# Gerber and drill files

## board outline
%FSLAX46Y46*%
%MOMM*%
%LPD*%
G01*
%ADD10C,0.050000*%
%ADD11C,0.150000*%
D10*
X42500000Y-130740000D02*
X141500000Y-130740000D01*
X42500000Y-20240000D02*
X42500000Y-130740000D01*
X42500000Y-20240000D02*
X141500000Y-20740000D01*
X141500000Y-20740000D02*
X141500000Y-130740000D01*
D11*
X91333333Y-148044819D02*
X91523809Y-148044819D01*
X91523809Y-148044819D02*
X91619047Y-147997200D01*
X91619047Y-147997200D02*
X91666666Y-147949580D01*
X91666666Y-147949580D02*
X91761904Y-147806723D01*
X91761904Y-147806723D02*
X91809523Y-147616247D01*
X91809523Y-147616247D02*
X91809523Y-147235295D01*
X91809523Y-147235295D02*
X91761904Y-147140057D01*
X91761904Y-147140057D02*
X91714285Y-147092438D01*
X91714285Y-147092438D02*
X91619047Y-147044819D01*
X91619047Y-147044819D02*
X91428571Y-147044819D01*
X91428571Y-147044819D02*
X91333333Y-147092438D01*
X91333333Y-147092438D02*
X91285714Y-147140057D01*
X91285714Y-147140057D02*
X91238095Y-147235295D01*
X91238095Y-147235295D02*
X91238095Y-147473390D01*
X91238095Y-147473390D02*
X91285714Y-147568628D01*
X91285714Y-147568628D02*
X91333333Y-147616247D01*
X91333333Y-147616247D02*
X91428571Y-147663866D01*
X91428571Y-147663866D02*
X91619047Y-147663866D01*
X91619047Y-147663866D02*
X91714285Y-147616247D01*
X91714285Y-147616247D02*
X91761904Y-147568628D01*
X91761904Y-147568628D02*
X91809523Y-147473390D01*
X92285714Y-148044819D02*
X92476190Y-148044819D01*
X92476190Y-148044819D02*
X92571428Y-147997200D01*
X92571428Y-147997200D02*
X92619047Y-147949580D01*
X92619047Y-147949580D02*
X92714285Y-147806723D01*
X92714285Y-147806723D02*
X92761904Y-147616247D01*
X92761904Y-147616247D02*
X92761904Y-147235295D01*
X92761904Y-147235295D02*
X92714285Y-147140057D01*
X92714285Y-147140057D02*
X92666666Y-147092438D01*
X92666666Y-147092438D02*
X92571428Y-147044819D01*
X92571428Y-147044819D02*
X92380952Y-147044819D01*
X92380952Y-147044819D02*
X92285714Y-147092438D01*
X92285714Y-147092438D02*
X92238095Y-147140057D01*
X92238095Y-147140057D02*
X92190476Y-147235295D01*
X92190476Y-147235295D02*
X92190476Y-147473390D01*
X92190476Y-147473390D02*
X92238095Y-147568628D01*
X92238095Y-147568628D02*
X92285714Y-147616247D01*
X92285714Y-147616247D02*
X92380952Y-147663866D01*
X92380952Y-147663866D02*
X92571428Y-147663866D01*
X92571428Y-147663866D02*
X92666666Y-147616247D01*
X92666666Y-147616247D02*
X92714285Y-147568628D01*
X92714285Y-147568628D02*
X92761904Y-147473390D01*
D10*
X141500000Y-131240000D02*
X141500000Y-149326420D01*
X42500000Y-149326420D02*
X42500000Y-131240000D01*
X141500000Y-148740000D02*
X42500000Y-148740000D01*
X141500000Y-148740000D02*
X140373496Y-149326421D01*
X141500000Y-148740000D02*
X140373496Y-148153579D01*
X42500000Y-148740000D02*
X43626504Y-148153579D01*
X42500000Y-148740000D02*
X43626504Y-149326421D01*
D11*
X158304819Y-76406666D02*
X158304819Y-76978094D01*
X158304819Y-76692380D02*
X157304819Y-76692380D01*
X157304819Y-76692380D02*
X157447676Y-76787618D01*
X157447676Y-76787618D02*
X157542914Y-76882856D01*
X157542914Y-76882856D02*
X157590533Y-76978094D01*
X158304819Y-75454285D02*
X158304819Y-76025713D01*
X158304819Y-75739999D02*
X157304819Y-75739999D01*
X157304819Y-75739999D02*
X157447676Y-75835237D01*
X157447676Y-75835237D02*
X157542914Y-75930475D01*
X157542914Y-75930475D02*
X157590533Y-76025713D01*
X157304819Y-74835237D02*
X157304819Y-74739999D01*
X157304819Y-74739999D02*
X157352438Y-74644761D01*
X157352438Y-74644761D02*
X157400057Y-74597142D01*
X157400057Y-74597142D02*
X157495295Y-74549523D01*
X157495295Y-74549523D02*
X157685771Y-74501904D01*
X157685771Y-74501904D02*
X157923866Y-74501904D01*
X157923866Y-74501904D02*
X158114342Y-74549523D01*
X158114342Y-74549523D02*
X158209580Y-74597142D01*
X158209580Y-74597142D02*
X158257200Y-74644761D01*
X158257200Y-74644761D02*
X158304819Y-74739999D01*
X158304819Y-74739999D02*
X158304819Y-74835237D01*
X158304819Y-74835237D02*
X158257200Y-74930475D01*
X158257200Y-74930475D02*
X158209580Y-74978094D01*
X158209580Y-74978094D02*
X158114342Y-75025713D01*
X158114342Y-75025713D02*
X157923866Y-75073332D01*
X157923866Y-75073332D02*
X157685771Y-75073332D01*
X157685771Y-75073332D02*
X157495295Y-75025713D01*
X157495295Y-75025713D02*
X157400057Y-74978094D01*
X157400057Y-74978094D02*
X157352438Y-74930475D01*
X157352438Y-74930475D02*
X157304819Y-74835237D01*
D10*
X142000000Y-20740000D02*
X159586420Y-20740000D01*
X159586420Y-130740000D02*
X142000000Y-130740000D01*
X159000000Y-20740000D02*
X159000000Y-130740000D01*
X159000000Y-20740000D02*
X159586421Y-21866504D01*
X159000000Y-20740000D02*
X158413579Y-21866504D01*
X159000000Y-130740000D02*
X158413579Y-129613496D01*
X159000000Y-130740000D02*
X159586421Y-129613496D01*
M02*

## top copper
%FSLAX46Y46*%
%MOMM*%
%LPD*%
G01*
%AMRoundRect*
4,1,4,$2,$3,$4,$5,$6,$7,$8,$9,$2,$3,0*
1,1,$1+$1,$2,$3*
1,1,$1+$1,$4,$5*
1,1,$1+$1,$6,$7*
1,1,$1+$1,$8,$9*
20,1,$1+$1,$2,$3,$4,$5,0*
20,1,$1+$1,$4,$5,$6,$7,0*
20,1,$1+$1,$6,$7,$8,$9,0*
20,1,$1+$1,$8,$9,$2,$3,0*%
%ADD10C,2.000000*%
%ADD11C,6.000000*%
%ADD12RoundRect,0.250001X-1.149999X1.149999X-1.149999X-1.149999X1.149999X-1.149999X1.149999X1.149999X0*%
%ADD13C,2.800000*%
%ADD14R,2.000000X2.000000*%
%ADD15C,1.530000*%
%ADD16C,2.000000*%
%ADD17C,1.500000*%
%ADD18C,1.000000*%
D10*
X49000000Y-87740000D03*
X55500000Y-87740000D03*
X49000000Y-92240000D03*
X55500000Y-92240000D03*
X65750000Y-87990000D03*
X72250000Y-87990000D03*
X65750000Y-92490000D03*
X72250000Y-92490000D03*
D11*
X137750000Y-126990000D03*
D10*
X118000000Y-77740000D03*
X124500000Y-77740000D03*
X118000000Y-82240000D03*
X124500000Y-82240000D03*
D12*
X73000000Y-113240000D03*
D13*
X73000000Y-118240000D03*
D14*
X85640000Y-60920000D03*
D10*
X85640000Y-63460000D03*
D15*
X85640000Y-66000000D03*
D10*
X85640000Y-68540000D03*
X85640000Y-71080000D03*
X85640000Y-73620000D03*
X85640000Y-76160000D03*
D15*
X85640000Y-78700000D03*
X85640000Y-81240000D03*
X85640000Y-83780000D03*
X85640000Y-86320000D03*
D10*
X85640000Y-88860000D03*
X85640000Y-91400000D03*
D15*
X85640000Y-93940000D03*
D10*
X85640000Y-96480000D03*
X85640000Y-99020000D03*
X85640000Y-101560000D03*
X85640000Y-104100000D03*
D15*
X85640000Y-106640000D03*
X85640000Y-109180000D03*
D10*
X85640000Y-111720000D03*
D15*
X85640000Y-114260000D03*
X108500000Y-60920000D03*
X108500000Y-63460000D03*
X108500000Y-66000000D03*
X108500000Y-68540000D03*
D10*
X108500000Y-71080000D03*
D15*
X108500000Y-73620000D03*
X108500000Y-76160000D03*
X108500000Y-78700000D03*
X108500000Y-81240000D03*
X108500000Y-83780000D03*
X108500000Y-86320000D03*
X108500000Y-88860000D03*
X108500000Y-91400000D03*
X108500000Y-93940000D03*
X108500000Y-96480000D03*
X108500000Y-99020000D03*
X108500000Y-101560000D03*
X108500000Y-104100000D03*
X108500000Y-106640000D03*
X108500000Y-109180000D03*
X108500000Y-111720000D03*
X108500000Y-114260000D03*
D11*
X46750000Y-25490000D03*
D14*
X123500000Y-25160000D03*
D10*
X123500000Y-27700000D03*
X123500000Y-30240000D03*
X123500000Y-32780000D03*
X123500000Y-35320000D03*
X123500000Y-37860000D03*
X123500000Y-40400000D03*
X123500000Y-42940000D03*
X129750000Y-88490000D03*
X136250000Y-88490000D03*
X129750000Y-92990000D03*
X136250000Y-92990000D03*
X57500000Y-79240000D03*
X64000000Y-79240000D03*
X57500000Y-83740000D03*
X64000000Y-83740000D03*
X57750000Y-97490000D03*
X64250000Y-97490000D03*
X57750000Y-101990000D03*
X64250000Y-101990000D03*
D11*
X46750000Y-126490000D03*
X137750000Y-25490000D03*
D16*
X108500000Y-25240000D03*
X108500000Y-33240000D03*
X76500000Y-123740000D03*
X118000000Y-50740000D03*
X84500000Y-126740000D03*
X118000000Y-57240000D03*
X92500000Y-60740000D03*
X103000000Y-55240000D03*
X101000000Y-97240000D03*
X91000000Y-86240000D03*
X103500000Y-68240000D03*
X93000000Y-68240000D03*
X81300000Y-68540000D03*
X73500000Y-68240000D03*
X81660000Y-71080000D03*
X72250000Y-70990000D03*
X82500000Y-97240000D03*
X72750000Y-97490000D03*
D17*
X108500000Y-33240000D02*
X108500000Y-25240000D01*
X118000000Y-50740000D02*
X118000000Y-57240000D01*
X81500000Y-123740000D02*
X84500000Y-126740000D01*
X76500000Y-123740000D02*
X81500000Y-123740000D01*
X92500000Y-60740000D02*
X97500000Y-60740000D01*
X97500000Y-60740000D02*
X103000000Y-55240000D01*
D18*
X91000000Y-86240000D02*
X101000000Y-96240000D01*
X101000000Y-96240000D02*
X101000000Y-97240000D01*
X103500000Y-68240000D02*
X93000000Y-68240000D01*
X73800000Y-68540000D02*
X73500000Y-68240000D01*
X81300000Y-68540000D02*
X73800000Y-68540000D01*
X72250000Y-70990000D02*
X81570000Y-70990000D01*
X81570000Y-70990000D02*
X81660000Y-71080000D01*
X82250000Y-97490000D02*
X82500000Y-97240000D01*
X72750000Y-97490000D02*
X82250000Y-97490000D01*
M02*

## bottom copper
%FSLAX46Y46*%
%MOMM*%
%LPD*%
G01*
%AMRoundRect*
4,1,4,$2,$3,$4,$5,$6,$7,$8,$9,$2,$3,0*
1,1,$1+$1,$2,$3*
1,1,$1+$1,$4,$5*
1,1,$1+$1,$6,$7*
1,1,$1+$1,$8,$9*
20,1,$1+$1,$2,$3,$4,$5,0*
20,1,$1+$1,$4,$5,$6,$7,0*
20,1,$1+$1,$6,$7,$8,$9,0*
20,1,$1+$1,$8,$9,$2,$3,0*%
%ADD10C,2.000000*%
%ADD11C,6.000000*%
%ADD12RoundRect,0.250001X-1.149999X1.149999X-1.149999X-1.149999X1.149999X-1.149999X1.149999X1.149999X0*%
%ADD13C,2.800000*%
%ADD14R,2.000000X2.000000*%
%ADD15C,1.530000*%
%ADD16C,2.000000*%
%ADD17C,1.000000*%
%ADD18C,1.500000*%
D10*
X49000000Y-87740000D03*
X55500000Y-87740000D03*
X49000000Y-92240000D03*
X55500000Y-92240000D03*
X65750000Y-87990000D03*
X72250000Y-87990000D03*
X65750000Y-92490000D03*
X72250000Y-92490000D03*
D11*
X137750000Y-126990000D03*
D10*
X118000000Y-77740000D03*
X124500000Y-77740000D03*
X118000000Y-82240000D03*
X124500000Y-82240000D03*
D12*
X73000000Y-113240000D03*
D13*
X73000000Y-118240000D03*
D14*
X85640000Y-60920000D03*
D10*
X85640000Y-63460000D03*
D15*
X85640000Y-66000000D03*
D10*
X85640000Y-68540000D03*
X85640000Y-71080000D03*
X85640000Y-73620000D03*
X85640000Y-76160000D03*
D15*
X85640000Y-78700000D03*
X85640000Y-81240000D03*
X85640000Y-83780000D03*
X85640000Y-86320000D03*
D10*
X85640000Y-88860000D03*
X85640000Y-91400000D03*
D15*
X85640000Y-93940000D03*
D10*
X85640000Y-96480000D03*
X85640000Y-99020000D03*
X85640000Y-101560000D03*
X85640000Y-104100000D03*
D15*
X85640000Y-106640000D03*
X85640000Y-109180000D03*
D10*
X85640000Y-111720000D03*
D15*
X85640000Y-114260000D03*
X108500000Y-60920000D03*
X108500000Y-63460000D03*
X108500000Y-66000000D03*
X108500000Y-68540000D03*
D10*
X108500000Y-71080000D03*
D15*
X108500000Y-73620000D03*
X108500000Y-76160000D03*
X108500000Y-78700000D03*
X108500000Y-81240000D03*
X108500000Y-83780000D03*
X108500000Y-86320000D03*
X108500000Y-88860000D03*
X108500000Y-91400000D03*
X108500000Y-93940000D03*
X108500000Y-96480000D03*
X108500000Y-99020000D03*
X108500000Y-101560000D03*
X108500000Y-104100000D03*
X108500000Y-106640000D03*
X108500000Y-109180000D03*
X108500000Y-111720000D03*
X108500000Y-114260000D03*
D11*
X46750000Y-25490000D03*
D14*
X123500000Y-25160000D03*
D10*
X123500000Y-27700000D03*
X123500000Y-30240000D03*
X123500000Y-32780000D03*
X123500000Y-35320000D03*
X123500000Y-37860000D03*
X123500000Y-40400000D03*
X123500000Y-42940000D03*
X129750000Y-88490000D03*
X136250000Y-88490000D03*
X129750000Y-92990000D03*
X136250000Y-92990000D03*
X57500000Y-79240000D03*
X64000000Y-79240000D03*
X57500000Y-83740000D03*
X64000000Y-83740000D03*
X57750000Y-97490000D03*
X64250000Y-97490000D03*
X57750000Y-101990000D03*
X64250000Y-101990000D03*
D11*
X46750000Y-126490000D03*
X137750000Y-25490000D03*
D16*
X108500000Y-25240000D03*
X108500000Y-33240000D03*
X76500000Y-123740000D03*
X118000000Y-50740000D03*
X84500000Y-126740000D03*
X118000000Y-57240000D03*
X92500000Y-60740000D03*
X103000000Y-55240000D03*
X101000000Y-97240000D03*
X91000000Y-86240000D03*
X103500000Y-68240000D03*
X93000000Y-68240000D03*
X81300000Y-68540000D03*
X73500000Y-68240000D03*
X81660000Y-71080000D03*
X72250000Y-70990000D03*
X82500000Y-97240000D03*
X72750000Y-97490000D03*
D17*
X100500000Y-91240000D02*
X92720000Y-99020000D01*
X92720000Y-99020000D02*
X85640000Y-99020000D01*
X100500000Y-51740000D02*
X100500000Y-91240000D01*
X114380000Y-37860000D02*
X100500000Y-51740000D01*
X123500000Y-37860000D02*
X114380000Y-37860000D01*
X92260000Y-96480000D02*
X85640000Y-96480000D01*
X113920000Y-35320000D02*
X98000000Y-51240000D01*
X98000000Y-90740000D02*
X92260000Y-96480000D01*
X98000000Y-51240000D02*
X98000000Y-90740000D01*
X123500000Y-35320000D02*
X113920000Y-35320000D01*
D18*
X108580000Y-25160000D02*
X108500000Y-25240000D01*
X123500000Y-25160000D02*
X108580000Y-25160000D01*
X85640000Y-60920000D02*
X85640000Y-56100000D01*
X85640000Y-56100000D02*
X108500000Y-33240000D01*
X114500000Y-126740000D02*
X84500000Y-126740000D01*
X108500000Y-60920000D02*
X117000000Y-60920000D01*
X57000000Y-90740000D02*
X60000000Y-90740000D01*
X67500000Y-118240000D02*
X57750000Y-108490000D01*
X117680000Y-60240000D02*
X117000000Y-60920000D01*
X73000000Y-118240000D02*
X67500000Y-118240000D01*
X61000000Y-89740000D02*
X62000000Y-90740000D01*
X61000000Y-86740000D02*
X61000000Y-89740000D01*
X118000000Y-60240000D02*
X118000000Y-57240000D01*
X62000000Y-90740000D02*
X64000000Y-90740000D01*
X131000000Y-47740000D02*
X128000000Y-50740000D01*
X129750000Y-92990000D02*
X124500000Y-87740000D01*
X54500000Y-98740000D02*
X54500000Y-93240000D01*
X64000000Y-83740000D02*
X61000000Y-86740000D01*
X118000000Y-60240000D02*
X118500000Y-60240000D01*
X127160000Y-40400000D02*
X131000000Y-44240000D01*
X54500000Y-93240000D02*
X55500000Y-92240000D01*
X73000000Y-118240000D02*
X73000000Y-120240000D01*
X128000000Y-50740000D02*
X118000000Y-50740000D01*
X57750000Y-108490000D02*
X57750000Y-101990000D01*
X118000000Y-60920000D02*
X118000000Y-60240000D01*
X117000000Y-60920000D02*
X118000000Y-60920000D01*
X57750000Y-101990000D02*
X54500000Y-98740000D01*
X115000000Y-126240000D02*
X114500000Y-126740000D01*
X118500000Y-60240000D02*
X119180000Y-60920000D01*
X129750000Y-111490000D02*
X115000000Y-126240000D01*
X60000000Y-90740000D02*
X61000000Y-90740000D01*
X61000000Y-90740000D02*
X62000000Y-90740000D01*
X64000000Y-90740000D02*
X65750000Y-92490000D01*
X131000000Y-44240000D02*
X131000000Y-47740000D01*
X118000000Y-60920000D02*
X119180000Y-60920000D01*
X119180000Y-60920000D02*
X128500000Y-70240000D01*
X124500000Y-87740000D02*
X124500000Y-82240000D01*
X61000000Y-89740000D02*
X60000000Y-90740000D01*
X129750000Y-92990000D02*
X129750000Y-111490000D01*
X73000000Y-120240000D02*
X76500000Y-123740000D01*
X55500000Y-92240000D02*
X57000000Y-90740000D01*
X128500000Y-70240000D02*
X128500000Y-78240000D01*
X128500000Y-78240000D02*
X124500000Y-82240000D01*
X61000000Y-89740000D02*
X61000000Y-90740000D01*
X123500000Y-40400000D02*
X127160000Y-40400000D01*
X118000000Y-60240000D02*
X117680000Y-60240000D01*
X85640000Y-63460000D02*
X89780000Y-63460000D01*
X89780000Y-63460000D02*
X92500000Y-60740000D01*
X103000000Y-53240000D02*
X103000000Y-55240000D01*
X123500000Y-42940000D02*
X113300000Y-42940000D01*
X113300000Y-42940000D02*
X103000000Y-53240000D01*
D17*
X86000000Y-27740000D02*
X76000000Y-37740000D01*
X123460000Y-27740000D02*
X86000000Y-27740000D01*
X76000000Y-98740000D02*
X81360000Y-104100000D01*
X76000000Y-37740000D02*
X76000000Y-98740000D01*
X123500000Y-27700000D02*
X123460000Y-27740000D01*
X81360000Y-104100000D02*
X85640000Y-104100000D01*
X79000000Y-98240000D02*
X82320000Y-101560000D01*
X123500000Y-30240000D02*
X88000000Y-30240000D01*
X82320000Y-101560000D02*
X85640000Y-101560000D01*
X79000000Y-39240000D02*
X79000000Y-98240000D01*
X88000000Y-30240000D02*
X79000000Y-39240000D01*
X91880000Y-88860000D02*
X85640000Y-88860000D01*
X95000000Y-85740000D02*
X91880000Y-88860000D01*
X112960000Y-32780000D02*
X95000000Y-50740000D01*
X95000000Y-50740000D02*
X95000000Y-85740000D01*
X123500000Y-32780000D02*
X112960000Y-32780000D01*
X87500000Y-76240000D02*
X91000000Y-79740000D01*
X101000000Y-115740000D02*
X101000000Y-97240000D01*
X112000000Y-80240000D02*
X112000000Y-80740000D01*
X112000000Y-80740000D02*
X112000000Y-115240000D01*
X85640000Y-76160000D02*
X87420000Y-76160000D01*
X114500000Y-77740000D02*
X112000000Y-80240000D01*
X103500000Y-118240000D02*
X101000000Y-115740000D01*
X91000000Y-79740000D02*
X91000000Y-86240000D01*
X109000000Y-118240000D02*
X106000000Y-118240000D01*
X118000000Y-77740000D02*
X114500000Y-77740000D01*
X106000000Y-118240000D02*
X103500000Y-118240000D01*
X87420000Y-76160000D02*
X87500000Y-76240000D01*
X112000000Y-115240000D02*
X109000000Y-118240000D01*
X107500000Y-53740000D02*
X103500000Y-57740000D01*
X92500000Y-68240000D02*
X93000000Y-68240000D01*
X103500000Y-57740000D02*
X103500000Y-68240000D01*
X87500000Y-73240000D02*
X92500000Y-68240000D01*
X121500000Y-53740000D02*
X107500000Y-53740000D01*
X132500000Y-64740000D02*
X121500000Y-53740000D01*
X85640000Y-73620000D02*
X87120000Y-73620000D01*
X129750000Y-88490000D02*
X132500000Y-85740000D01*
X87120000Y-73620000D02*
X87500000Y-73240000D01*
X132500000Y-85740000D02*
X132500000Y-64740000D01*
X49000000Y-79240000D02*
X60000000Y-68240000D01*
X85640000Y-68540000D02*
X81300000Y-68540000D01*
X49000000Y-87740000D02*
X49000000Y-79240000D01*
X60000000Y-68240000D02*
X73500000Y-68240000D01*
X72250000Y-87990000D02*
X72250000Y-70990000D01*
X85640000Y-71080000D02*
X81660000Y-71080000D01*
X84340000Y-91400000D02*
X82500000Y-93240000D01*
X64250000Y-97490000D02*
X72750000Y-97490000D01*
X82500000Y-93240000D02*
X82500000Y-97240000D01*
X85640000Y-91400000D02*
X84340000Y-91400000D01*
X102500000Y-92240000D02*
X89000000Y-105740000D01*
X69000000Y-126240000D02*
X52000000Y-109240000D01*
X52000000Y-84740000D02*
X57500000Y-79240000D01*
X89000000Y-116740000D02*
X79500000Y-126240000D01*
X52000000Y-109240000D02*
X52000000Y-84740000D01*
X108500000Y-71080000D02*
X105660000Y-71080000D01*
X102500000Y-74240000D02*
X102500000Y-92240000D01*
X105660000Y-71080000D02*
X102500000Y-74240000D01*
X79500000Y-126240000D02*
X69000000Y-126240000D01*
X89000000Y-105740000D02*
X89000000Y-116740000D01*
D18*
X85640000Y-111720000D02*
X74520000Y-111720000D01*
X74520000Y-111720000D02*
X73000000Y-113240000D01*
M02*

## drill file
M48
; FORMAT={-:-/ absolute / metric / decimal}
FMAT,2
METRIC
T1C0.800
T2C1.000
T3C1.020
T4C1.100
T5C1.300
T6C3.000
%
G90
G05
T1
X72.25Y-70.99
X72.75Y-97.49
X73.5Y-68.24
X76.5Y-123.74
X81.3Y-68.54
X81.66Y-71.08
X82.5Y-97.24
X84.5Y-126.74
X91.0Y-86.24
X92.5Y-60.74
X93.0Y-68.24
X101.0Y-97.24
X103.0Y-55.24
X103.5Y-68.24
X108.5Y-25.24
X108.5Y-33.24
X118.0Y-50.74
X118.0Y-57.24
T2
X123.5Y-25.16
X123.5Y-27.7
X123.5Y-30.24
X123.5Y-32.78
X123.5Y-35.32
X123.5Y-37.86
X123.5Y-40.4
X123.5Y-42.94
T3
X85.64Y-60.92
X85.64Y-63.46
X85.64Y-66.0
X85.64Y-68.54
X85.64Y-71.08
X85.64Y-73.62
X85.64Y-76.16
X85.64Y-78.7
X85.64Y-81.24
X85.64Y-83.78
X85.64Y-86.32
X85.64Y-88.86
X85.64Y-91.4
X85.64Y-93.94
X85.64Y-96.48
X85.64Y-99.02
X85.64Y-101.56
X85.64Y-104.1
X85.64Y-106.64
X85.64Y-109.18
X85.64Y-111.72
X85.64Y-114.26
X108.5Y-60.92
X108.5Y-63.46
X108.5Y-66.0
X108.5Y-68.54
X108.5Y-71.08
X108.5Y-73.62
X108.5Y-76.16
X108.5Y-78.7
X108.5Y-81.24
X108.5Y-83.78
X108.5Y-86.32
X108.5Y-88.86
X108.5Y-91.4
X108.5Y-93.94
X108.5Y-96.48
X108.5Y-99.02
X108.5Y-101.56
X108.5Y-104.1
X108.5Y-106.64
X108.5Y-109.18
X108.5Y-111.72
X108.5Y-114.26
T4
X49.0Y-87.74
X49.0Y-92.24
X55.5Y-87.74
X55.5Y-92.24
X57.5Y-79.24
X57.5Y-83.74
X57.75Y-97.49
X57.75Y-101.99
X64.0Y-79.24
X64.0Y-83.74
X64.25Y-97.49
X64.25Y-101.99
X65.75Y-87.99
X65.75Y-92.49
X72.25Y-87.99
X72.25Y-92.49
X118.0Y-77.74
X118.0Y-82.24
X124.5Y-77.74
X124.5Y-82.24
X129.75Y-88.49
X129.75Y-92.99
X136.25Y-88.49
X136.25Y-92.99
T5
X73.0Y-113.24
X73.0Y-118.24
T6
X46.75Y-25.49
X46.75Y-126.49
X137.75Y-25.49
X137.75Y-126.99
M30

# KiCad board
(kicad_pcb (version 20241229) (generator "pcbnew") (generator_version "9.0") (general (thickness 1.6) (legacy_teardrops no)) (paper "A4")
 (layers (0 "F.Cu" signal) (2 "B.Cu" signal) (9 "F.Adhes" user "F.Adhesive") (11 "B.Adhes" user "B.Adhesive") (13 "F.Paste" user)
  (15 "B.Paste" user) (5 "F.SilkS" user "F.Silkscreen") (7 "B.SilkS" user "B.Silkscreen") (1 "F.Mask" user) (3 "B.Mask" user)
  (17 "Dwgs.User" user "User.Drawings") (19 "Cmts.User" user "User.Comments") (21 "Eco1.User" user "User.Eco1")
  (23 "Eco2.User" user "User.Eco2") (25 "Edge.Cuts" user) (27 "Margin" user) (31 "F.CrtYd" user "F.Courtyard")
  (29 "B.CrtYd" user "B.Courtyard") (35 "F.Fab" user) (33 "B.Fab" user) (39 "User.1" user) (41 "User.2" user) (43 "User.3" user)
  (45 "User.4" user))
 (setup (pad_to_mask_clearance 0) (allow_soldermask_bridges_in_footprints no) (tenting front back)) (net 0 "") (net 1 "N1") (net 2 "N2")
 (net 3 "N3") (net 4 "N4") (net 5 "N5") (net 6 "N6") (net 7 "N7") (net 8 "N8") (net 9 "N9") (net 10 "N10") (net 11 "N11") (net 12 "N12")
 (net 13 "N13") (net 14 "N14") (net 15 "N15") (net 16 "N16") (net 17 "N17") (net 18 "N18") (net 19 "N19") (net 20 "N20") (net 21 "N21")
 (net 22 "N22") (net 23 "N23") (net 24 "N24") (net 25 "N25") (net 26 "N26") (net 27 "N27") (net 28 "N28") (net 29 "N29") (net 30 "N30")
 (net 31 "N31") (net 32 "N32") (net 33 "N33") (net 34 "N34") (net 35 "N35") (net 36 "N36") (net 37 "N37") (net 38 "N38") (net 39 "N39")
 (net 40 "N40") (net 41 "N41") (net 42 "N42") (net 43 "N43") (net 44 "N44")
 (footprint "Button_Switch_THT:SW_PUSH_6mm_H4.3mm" (layer "F.Cu") (at 49 87.74)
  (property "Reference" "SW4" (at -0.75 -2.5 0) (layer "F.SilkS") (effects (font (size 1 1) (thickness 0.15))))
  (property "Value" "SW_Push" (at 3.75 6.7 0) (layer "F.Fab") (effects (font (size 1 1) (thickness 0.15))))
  (pad "1" thru_hole circle (at 0 0 90) (size 2 2) (drill 1.1) (layers "*.Cu" "*.Mask") (remove_unused_layers no) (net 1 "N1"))
  (pad "1" thru_hole circle (at 6.5 0 90) (size 2 2) (drill 1.1) (layers "*.Cu" "*.Mask") (remove_unused_layers no) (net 1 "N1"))
  (pad "2" thru_hole circle (at 0 4.5 90) (size 2 2) (drill 1.1) (layers "*.Cu" "*.Mask") (remove_unused_layers no) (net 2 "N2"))
  (pad "2" thru_hole circle (at 6.5 4.5 90) (size 2 2) (drill 1.1) (layers "*.Cu" "*.Mask") (remove_unused_layers no) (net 2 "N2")))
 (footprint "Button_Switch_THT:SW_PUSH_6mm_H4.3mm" (layer "F.Cu") (at 65.75 87.99)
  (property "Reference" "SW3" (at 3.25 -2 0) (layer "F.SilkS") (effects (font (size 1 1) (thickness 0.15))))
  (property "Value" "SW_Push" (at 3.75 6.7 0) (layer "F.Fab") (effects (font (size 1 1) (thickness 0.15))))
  (pad "1" thru_hole circle (at 0 0 90) (size 2 2) (drill 1.1) (layers "*.Cu" "*.Mask") (remove_unused_layers no) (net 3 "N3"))
  (pad "1" thru_hole circle (at 6.5 0 90) (size 2 2) (drill 1.1) (layers "*.Cu" "*.Mask") (remove_unused_layers no) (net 3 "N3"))
  (pad "2" thru_hole circle (at 0 4.5 90) (size 2 2) (drill 1.1) (layers "*.Cu" "*.Mask") (remove_unused_layers no) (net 2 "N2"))
  (pad "2" thru_hole circle (at 6.5 4.5 90) (size 2 2) (drill 1.1) (layers "*.Cu" "*.Mask") (remove_unused_layers no) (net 2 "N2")))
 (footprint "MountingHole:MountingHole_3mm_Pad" (layer "F.Cu") (at 137.75 126.99)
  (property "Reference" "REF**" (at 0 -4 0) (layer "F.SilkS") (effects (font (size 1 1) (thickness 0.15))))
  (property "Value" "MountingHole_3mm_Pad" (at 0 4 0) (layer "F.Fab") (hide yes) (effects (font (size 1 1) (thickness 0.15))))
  (pad "1" thru_hole circle (at 0 0) (size 6 6) (drill 3) (layers "*.Cu" "*.Mask") (remove_unused_layers no)))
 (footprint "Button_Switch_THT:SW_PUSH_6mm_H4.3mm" (layer "F.Cu") (at 118 77.74)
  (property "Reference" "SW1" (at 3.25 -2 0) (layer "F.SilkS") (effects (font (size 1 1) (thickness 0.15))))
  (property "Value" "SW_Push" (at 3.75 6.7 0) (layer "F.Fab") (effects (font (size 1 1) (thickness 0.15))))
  (pad "1" thru_hole circle (at 0 0 90) (size 2 2) (drill 1.1) (layers "*.Cu" "*.Mask") (remove_unused_layers no) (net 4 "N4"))
  (pad "1" thru_hole circle (at 6.5 0 90) (size 2 2) (drill 1.1) (layers "*.Cu" "*.Mask") (remove_unused_layers no) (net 4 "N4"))
  (pad "2" thru_hole circle (at 0 4.5 90) (size 2 2) (drill 1.1) (layers "*.Cu" "*.Mask") (remove_unused_layers no) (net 2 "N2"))
  (pad "2" thru_hole circle (at 6.5 4.5 90) (size 2 2) (drill 1.1) (layers "*.Cu" "*.Mask") (remove_unused_layers no) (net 2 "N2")))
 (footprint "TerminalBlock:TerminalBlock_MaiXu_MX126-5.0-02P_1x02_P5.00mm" (layer "F.Cu") (at 73 113.24 -90)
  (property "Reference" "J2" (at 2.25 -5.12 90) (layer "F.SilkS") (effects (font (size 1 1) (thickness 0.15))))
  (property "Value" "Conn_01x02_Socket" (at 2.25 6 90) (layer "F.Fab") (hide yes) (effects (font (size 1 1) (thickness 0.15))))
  (pad "1" thru_hole roundrect (at 0 0 270) (size 2.8 2.8) (drill 1.3) (layers "*.Cu" "*.Mask") (remove_unused_layers no)
   (roundrect_rratio 0.089286) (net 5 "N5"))
  (pad "2" thru_hole circle (at 5 0 270) (size 2.8 2.8) (drill 1.3) (layers "*.Cu" "*.Mask") (remove_unused_layers no) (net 2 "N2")))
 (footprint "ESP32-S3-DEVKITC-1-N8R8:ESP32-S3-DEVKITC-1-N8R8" (layer "F.Cu") (at 97.07 90.89)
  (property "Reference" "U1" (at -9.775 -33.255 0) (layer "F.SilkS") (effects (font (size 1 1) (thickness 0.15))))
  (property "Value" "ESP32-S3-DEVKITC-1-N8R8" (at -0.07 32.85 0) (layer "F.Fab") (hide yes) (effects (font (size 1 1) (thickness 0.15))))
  (pad "J1_1" thru_hole rect (at -11.43 -29.97) (size 2 2) (drill 1.02) (layers "*.Cu" "*.Mask") (remove_unused_layers no) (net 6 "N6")
   (solder_mask_margin 0.102))
  (pad "J1_2" thru_hole circle (at -11.43 -27.43) (size 2 2) (drill 1.02) (layers "*.Cu" "*.Mask") (remove_unused_layers no) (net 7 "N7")
   (solder_mask_margin 0.102))
  (pad "J1_3" thru_hole circle (at -11.43 -24.89) (size 1.53 1.53) (drill 1.02) (layers "*.Cu" "*.Mask") (remove_unused_layers no)
   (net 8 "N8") (solder_mask_margin 0.102))
  (pad "J1_4" thru_hole circle (at -11.43 -22.35) (size 2 2) (drill 1.02) (layers "*.Cu" "*.Mask") (remove_unused_layers no) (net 1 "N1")
   (solder_mask_margin 0.102))
  (pad "J1_5" thru_hole circle (at -11.43 -19.81) (size 2 2) (drill 1.02) (layers "*.Cu" "*.Mask") (remove_unused_layers no) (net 3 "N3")
   (solder_mask_margin 0.102))
  (pad "J1_6" thru_hole circle (at -11.43 -17.27) (size 2 2) (drill 1.02) (layers "*.Cu" "*.Mask") (remove_unused_layers no) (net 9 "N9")
   (solder_mask_margin 0.102))
  (pad "J1_7" thru_hole circle (at -11.43 -14.73) (size 2 2) (drill 1.02) (layers "*.Cu" "*.Mask") (remove_unused_layers no) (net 4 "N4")
   (solder_mask_margin 0.102))
  (pad "J1_8" thru_hole circle (at -11.43 -12.19) (size 1.53 1.53) (drill 1.02) (layers "*.Cu" "*.Mask") (remove_unused_layers no)
   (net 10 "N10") (solder_mask_margin 0.102))
  (pad "J1_9" thru_hole circle (at -11.43 -9.65) (size 1.53 1.53) (drill 1.02) (layers "*.Cu" "*.Mask") (remove_unused_layers no)
   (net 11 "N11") (solder_mask_margin 0.102))
  (pad "J1_10" thru_hole circle (at -11.43 -7.11) (size 1.53 1.53) (drill 1.02) (layers "*.Cu" "*.Mask") (remove_unused_layers no)
   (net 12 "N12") (solder_mask_margin 0.102))
  (pad "J1_11" thru_hole circle (at -11.43 -4.57) (size 1.53 1.53) (drill 1.02) (layers "*.Cu" "*.Mask") (remove_unused_layers no)
   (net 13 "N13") (solder_mask_margin 0.102))
  (pad "J1_12" thru_hole circle (at -11.43 -2.03) (size 2 2) (drill 1.02) (layers "*.Cu" "*.Mask") (remove_unused_layers no) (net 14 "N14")
   (solder_mask_margin 0.102))
  (pad "J1_13" thru_hole circle (at -11.43 0.51) (size 2 2) (drill 1.02) (layers "*.Cu" "*.Mask") (remove_unused_layers no) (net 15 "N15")
   (solder_mask_margin 0.102))
  (pad "J1_14" thru_hole circle (at -11.43 3.05) (size 1.53 1.53) (drill 1.02) (layers "*.Cu" "*.Mask") (remove_unused_layers no)
   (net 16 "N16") (solder_mask_margin 0.102))
  (pad "J1_15" thru_hole circle (at -11.43 5.59) (size 2 2) (drill 1.02) (layers "*.Cu" "*.Mask") (remove_unused_layers no) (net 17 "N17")
   (solder_mask_margin 0.102))
  (pad "J1_16" thru_hole circle (at -11.43 8.13) (size 2 2) (drill 1.02) (layers "*.Cu" "*.Mask") (remove_unused_layers no) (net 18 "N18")
   (solder_mask_margin 0.102))
  (pad "J1_17" thru_hole circle (at -11.43 10.67) (size 2 2) (drill 1.02) (layers "*.Cu" "*.Mask") (remove_unused_layers no) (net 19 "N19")
   (solder_mask_margin 0.102))
  (pad "J1_18" thru_hole circle (at -11.43 13.21) (size 2 2) (drill 1.02) (layers "*.Cu" "*.Mask") (remove_unused_layers no) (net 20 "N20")
   (solder_mask_margin 0.102))
  (pad "J1_19" thru_hole circle (at -11.43 15.75) (size 1.53 1.53) (drill 1.02) (layers "*.Cu" "*.Mask") (remove_unused_layers no)
   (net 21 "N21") (solder_mask_margin 0.102))
  (pad "J1_20" thru_hole circle (at -11.43 18.29) (size 1.53 1.53) (drill 1.02) (layers "*.Cu" "*.Mask") (remove_unused_layers no)
   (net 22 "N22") (solder_mask_margin 0.102))
  (pad "J1_21" thru_hole circle (at -11.43 20.83) (size 2 2) (drill 1.02) (layers "*.Cu" "*.Mask") (remove_unused_layers no) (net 5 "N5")
   (solder_mask_margin 0.102))
  (pad "J1_22" thru_hole circle (at -11.43 23.37) (size 1.53 1.53) (drill 1.02) (layers "*.Cu" "*.Mask") (remove_unused_layers no)
   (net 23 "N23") (solder_mask_margin 0.102))
  (pad "J3_1" thru_hole circle (at 11.43 -29.97) (size 1.53 1.53) (drill 1.02) (layers "*.Cu" "*.Mask") (remove_unused_layers no)
   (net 2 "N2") (solder_mask_margin 0.102))
  (pad "J3_2" thru_hole circle (at 11.43 -27.43) (size 1.53 1.53) (drill 1.02) (layers "*.Cu" "*.Mask") (remove_unused_layers no)
   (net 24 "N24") (solder_mask_margin 0.102))
  (pad "J3_3" thru_hole circle (at 11.43 -24.89) (size 1.53 1.53) (drill 1.02) (layers "*.Cu" "*.Mask") (remove_unused_layers no)
   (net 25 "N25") (solder_mask_margin 0.102))
  (pad "J3_4" thru_hole circle (at 11.43 -22.35) (size 1.53 1.53) (drill 1.02) (layers "*.Cu" "*.Mask") (remove_unused_layers no)
   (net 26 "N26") (solder_mask_margin 0.102))
  (pad "J3_5" thru_hole circle (at 11.43 -19.81) (size 2 2) (drill 1.02) (layers "*.Cu" "*.Mask") (remove_unused_layers no) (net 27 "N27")
   (solder_mask_margin 0.102))
  (pad "J3_6" thru_hole circle (at 11.43 -17.27) (size 1.53 1.53) (drill 1.02) (layers "*.Cu" "*.Mask") (remove_unused_layers no)
   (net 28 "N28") (solder_mask_margin 0.102))
  (pad "J3_7" thru_hole circle (at 11.43 -14.73) (size 1.53 1.53) (drill 1.02) (layers "*.Cu" "*.Mask") (remove_unused_layers no)
   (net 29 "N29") (solder_mask_margin 0.102))
  (pad "J3_8" thru_hole circle (at 11.43 -12.19) (size 1.53 1.53) (drill 1.02) (layers "*.Cu" "*.Mask") (remove_unused_layers no)
   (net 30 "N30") (solder_mask_margin 0.102))
  (pad "J3_9" thru_hole circle (at 11.43 -9.65) (size 1.53 1.53) (drill 1.02) (layers "*.Cu" "*.Mask") (remove_unused_layers no)
   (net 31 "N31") (solder_mask_margin 0.102))
  (pad "J3_10" thru_hole circle (at 11.43 -7.11) (size 1.53 1.53) (drill 1.02) (layers "*.Cu" "*.Mask") (remove_unused_layers no)
   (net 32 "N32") (solder_mask_margin 0.102))
  (pad "J3_11" thru_hole circle (at 11.43 -4.57) (size 1.53 1.53) (drill 1.02) (layers "*.Cu" "*.Mask") (remove_unused_layers no)
   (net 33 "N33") (solder_mask_margin 0.102))
  (pad "J3_12" thru_hole circle (at 11.43 -2.03) (size 1.53 1.53) (drill 1.02) (layers "*.Cu" "*.Mask") (remove_unused_layers no)
   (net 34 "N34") (solder_mask_margin 0.102))
  (pad "J3_13" thru_hole circle (at 11.43 0.51) (size 1.53 1.53) (drill 1.02) (layers "*.Cu" "*.Mask") (remove_unused_layers no)
   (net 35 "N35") (solder_mask_margin 0.102))
  (pad "J3_14" thru_hole circle (at 11.43 3.05) (size 1.53 1.53) (drill 1.02) (layers "*.Cu" "*.Mask") (remove_unused_layers no)
   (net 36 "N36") (solder_mask_margin 0.102))
  (pad "J3_15" thru_hole circle (at 11.43 5.59) (size 1.53 1.53) (drill 1.02) (layers "*.Cu" "*.Mask") (remove_unused_layers no)
   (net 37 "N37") (solder_mask_margin 0.102))
  (pad "J3_16" thru_hole circle (at 11.43 8.13) (size 1.53 1.53) (drill 1.02) (layers "*.Cu" "*.Mask") (remove_unused_layers no)
   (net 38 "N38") (solder_mask_margin 0.102))
  (pad "J3_17" thru_hole circle (at 11.43 10.67) (size 1.53 1.53) (drill 1.02) (layers "*.Cu" "*.Mask") (remove_unused_layers no)
   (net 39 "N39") (solder_mask_margin 0.102))
  (pad "J3_18" thru_hole circle (at 11.43 13.21) (size 1.53 1.53) (drill 1.02) (layers "*.Cu" "*.Mask") (remove_unused_layers no)
   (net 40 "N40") (solder_mask_margin 0.102))
  (pad "J3_19" thru_hole circle (at 11.43 15.75) (size 1.53 1.53) (drill 1.02) (layers "*.Cu" "*.Mask") (remove_unused_layers no)
   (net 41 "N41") (solder_mask_margin 0.102))
  (pad "J3_20" thru_hole circle (at 11.43 18.29) (size 1.53 1.53) (drill 1.02) (layers "*.Cu" "*.Mask") (remove_unused_layers no)
   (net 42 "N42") (solder_mask_margin 0.102))
  (pad "J3_21" thru_hole circle (at 11.43 20.83) (size 1.53 1.53) (drill 1.02) (layers "*.Cu" "*.Mask") (remove_unused_layers no)
   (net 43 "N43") (solder_mask_margin 0.102))
  (pad "J3_22" thru_hole circle (at 11.43 23.37) (size 1.53 1.53) (drill 1.02) (layers "*.Cu" "*.Mask") (remove_unused_layers no)
   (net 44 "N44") (solder_mask_margin 0.102)))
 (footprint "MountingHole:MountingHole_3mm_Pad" (layer "F.Cu") (at 46.75 25.49)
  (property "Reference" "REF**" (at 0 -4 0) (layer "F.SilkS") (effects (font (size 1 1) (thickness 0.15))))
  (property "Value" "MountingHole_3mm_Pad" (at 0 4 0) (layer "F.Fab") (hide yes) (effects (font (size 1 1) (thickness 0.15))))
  (pad "1" thru_hole circle (at 0 0) (size 6 6) (drill 3) (layers "*.Cu" "*.Mask") (remove_unused_layers no)))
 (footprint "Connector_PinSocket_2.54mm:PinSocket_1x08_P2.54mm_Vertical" (layer "F.Cu") (at 123.5 25.16)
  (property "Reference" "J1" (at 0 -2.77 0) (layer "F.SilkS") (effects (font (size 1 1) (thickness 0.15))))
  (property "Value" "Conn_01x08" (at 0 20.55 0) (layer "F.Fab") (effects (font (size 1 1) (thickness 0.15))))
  (pad "1" thru_hole rect (at 0 0) (size 2 2) (drill 1) (layers "*.Cu" "*.Mask") (remove_unused_layers no) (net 6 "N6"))
  (pad "2" thru_hole circle (at 0 2.54) (size 2 2) (drill 1) (layers "*.Cu" "*.Mask") (remove_unused_layers no) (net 20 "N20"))
  (pad "3" thru_hole circle (at 0 5.08) (size 2 2) (drill 1) (layers "*.Cu" "*.Mask") (remove_unused_layers no) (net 19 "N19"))
  (pad "4" thru_hole circle (at 0 7.62) (size 2 2) (drill 1) (layers "*.Cu" "*.Mask") (remove_unused_layers no) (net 14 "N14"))
  (pad "5" thru_hole circle (at 0 10.16) (size 2 2) (drill 1) (layers "*.Cu" "*.Mask") (remove_unused_layers no) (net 17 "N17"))
  (pad "6" thru_hole circle (at 0 12.7) (size 2 2) (drill 1) (layers "*.Cu" "*.Mask") (remove_unused_layers no) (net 18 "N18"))
  (pad "7" thru_hole circle (at 0 15.24) (size 2 2) (drill 1) (layers "*.Cu" "*.Mask") (remove_unused_layers no) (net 2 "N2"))
  (pad "8" thru_hole circle (at 0 17.78) (size 2 2) (drill 1) (layers "*.Cu" "*.Mask") (remove_unused_layers no) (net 7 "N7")))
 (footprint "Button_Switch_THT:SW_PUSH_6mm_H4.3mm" (layer "F.Cu") (at 129.75 88.49)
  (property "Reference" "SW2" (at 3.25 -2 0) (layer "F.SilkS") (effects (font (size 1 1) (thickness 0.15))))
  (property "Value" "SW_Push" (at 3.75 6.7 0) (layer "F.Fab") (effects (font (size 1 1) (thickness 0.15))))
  (pad "1" thru_hole circle (at 0 0 90) (size 2 2) (drill 1.1) (layers "*.Cu" "*.Mask") (remove_unused_layers no) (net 9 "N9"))
  (pad "1" thru_hole circle (at 6.5 0 90) (size 2 2) (drill 1.1) (layers "*.Cu" "*.Mask") (remove_unused_layers no) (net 9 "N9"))
  (pad "2" thru_hole circle (at 0 4.5 90) (size 2 2) (drill 1.1) (layers "*.Cu" "*.Mask") (remove_unused_layers no) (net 2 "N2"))
  (pad "2" thru_hole circle (at 6.5 4.5 90) (size 2 2) (drill 1.1) (layers "*.Cu" "*.Mask") (remove_unused_layers no) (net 2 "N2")))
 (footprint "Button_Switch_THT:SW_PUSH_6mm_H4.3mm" (layer "F.Cu") (at 57.5 79.24)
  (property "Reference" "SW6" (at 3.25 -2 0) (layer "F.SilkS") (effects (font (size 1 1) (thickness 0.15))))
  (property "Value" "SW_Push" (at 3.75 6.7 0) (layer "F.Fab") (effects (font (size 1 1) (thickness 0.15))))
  (pad "1" thru_hole circle (at 0 0 90) (size 2 2) (drill 1.1) (layers "*.Cu" "*.Mask") (remove_unused_layers no) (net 27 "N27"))
  (pad "1" thru_hole circle (at 6.5 0 90) (size 2 2) (drill 1.1) (layers "*.Cu" "*.Mask") (remove_unused_layers no) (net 27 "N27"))
  (pad "2" thru_hole circle (at 0 4.5 90) (size 2 2) (drill 1.1) (layers "*.Cu" "*.Mask") (remove_unused_layers no) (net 2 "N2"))
  (pad "2" thru_hole circle (at 6.5 4.5 90) (size 2 2) (drill 1.1) (layers "*.Cu" "*.Mask") (remove_unused_layers no) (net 2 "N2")))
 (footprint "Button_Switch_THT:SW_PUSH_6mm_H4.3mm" (layer "F.Cu") (at 57.75 97.49)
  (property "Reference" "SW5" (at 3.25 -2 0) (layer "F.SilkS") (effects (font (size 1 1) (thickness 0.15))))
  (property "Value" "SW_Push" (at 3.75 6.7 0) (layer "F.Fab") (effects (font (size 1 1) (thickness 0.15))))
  (pad "1" thru_hole circle (at 0 0 90) (size 2 2) (drill 1.1) (layers "*.Cu" "*.Mask") (remove_unused_layers no) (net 15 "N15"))
  (pad "1" thru_hole circle (at 6.5 0 90) (size 2 2) (drill 1.1) (layers "*.Cu" "*.Mask") (remove_unused_layers no) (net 15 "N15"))
  (pad "2" thru_hole circle (at 0 4.5 90) (size 2 2) (drill 1.1) (layers "*.Cu" "*.Mask") (remove_unused_layers no) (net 2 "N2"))
  (pad "2" thru_hole circle (at 6.5 4.5 90) (size 2 2) (drill 1.1) (layers "*.Cu" "*.Mask") (remove_unused_layers no) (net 2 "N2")))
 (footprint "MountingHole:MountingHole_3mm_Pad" (layer "F.Cu") (at 46.75 126.49)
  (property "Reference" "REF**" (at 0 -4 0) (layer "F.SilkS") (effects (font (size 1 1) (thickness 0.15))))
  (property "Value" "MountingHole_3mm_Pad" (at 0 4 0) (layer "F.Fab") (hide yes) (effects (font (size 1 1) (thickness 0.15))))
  (pad "1" thru_hole circle (at 0 0) (size 6 6) (drill 3) (layers "*.Cu" "*.Mask") (remove_unused_layers no)))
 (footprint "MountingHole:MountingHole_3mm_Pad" (layer "F.Cu") (at 137.75 25.49)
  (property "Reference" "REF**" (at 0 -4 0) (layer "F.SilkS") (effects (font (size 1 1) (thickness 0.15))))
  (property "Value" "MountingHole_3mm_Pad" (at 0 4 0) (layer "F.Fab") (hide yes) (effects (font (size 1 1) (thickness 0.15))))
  (pad "1" thru_hole circle (at 0 0) (size 6 6) (drill 3) (layers "*.Cu" "*.Mask") (remove_unused_layers no)))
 (gr_line (start 42.5 130.74) (end 141.5 130.74) (stroke (width 0.05) (type default)) (layer "Edge.Cuts"))
 (gr_line (start 42.5 20.24) (end 42.5 130.74) (stroke (width 0.05) (type default)) (layer "Edge.Cuts"))
 (gr_line (start 42.5 20.24) (end 141.5 20.74) (stroke (width 0.05) (type default)) (layer "Edge.Cuts"))
 (gr_line (start 141.5 20.74) (end 141.5 130.74) (stroke (width 0.05) (type default)) (layer "Edge.Cuts"))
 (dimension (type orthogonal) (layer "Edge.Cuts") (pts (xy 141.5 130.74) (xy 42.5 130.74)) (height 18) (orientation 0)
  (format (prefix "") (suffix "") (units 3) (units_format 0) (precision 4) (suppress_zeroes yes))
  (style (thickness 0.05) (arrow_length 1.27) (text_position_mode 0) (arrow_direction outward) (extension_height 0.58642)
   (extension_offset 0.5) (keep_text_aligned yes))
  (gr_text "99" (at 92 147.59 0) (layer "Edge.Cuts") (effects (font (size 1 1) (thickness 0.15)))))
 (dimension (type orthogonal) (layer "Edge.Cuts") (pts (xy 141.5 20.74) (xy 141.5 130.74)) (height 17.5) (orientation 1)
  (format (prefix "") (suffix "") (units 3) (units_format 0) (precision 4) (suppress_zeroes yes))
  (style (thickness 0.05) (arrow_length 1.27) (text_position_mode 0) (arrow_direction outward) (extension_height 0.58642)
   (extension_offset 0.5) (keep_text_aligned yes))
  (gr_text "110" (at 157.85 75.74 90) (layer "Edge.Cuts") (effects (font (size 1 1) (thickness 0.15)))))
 (segment (start 100.5 91.24) (end 92.72 99.02) (width 1) (layer "B.Cu") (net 18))
 (segment (start 92.72 99.02) (end 85.64 99.02) (width 1) (layer "B.Cu") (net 18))
 (segment (start 100.5 51.74) (end 100.5 91.24) (width 1) (layer "B.Cu") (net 18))
 (segment (start 114.38 37.86) (end 100.5 51.74) (width 1) (layer "B.Cu") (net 18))
 (segment (start 123.5 37.86) (end 114.38 37.86) (width 1) (layer "B.Cu") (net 18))
 (segment (start 92.26 96.48) (end 85.64 96.48) (width 1) (layer "B.Cu") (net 17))
 (segment (start 113.92 35.32) (end 98 51.24) (width 1) (layer "B.Cu") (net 17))
 (segment (start 98 90.74) (end 92.26 96.48) (width 1) (layer "B.Cu") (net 17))
 (segment (start 98 51.24) (end 98 90.74) (width 1) (layer "B.Cu") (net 17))
 (segment (start 123.5 35.32) (end 113.92 35.32) (width 1) (layer "B.Cu") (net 17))
 (segment (start 108.5 33.24) (end 108.5 25.24) (width 1.5) (layer "F.Cu") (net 6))
 (via (at 108.5 25.24) (size 2) (drill 0.8) (layers "F.Cu" "B.Cu") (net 6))
 (via (at 108.5 33.24) (size 2) (drill 0.8) (layers "F.Cu" "B.Cu") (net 6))
 (segment (start 108.58 25.16) (end 108.5 25.24) (width 1.5) (layer "B.Cu") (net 6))
 (segment (start 123.5 25.16) (end 108.58 25.16) (width 1.5) (layer "B.Cu") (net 6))
 (segment (start 85.64 60.92) (end 85.64 56.1) (width 1.5) (layer "B.Cu") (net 6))
 (segment (start 85.64 56.1) (end 108.5 33.24) (width 1.5) (layer "B.Cu") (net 6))
 (segment (start 118 50.74) (end 118 57.24) (width 1.5) (layer "F.Cu") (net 2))
 (segment (start 81.5 123.74) (end 84.5 126.74) (width 1.5) (layer "F.Cu") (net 2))
 (segment (start 76.5 123.74) (end 81.5 123.74) (width 1.5) (layer "F.Cu") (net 2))
 (via (at 76.5 123.74) (size 2) (drill 0.8) (layers "F.Cu" "B.Cu") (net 2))
 (via (at 118 50.74) (size 2) (drill 0.8) (layers "F.Cu" "B.Cu") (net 2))
 (via (at 84.5 126.74) (size 2) (drill 0.8) (layers "F.Cu" "B.Cu") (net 2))
 (via (at 118 57.24) (size 2) (drill 0.8) (layers "F.Cu" "B.Cu") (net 2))
 (segment (start 114.5 126.74) (end 84.5 126.74) (width 1.5) (layer "B.Cu") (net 2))
 (segment (start 108.5 60.92) (end 117 60.92) (width 1.5) (layer "B.Cu") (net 2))
 (segment (start 57 90.74) (end 60 90.74) (width 1.5) (layer "B.Cu") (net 2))
 (segment (start 67.5 118.24) (end 57.75 108.49) (width 1.5) (layer "B.Cu") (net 2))
 (segment (start 117.68 60.24) (end 117 60.92) (width 1.5) (layer "B.Cu") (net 2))
 (segment (start 73 118.24) (end 67.5 118.24) (width 1.5) (layer "B.Cu") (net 2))
 (segment (start 61 89.74) (end 62 90.74) (width 1.5) (layer "B.Cu") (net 2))
 (segment (start 61 86.74) (end 61 89.74) (width 1.5) (layer "B.Cu") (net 2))
 (segment (start 118 60.24) (end 118 57.24) (width 1.5) (layer "B.Cu") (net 2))
 (segment (start 62 90.74) (end 64 90.74) (width 1.5) (layer "B.Cu") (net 2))
 (segment (start 131 47.74) (end 128 50.74) (width 1.5) (layer "B.Cu") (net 2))
 (segment (start 129.75 92.99) (end 124.5 87.74) (width 1.5) (layer "B.Cu") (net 2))
 (segment (start 54.5 98.74) (end 54.5 93.24) (width 1.5) (layer "B.Cu") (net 2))
 (segment (start 64 83.74) (end 61 86.74) (width 1.5) (layer "B.Cu") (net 2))
 (segment (start 118 60.24) (end 118.5 60.24) (width 1.5) (layer "B.Cu") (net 2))
 (segment (start 127.16 40.4) (end 131 44.24) (width 1.5) (layer "B.Cu") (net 2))
 (segment (start 54.5 93.24) (end 55.5 92.24) (width 1.5) (layer "B.Cu") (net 2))
 (segment (start 73 118.24) (end 73 120.24) (width 1.5) (layer "B.Cu") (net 2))
 (segment (start 128 50.74) (end 118 50.74) (width 1.5) (layer "B.Cu") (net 2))
 (segment (start 57.75 108.49) (end 57.75 101.99) (width 1.5) (layer "B.Cu") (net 2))
 (segment (start 118 60.92) (end 118 60.24) (width 1.5) (layer "B.Cu") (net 2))
 (segment (start 117 60.92) (end 118 60.92) (width 1.5) (layer "B.Cu") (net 2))
 (segment (start 57.75 101.99) (end 54.5 98.74) (width 1.5) (layer "B.Cu") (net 2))
 (segment (start 115 126.24) (end 114.5 126.74) (width 1.5) (layer "B.Cu") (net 2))
 (segment (start 118.5 60.24) (end 119.18 60.92) (width 1.5) (layer "B.Cu") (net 2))
 (segment (start 129.75 111.49) (end 115 126.24) (width 1.5) (layer "B.Cu") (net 2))
 (segment (start 60 90.74) (end 61 90.74) (width 1.5) (layer "B.Cu") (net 2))
 (segment (start 61 90.74) (end 62 90.74) (width 1.5) (layer "B.Cu") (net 2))
 (segment (start 64 90.74) (end 65.75 92.49) (width 1.5) (layer "B.Cu") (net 2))
 (segment (start 131 44.24) (end 131 47.74) (width 1.5) (layer "B.Cu") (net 2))
 (segment (start 118 60.92) (end 119.18 60.92) (width 1.5) (layer "B.Cu") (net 2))
 (segment (start 119.18 60.92) (end 128.5 70.24) (width 1.5) (layer "B.Cu") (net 2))
 (segment (start 124.5 87.74) (end 124.5 82.24) (width 1.5) (layer "B.Cu") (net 2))
 (segment (start 61 89.74) (end 60 90.74) (width 1.5) (layer "B.Cu") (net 2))
 (segment (start 129.75 92.99) (end 129.75 111.49) (width 1.5) (layer "B.Cu") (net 2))
 (segment (start 73 120.24) (end 76.5 123.74) (width 1.5) (layer "B.Cu") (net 2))
 (segment (start 55.5 92.24) (end 57 90.74) (width 1.5) (layer "B.Cu") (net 2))
 (segment (start 128.5 70.24) (end 128.5 78.24) (width 1.5) (layer "B.Cu") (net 2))
 (segment (start 128.5 78.24) (end 124.5 82.24) (width 1.5) (layer "B.Cu") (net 2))
 (segment (start 61 89.74) (end 61 90.74) (width 1.5) (layer "B.Cu") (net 2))
 (segment (start 123.5 40.4) (end 127.16 40.4) (width 1.5) (layer "B.Cu") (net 2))
 (segment (start 118 60.24) (end 117.68 60.24) (width 1.5) (layer "B.Cu") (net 2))
 (segment (start 92.5 60.74) (end 97.5 60.74) (width 1.5) (layer "F.Cu") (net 7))
 (segment (start 97.5 60.74) (end 103 55.24) (width 1.5) (layer "F.Cu") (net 7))
 (via (at 92.5 60.74) (size 2) (drill 0.8) (layers "F.Cu" "B.Cu") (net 7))
 (via (at 103 55.24) (size 2) (drill 0.8) (layers "F.Cu" "B.Cu") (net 7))
 (segment (start 85.64 63.46) (end 89.78 63.46) (width 1.5) (layer "B.Cu") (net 7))
 (segment (start 89.78 63.46) (end 92.5 60.74) (width 1.5) (layer "B.Cu") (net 7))
 (segment (start 103 53.24) (end 103 55.24) (width 1.5) (layer "B.Cu") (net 7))
 (segment (start 123.5 42.94) (end 113.3 42.94) (width 1.5) (layer "B.Cu") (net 7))
 (segment (start 113.3 42.94) (end 103 53.24) (width 1.5) (layer "B.Cu") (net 7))
 (segment (start 86 27.74) (end 76 37.74) (width 1) (layer "B.Cu") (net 20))
 (segment (start 123.46 27.74) (end 86 27.74) (width 1) (layer "B.Cu") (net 20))
 (segment (start 76 98.74) (end 81.36 104.1) (width 1) (layer "B.Cu") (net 20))
 (segment (start 76 37.74) (end 76 98.74) (width 1) (layer "B.Cu") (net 20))
 (segment (start 123.5 27.7) (end 123.46 27.74) (width 1) (layer "B.Cu") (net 20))
 (segment (start 81.36 104.1) (end 85.64 104.1) (width 1) (layer "B.Cu") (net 20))
 (segment (start 79 98.24) (end 82.32 101.56) (width 1) (layer "B.Cu") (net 19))
 (segment (start 123.5 30.24) (end 88 30.24) (width 1) (layer "B.Cu") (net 19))
 (segment (start 82.32 101.56) (end 85.64 101.56) (width 1) (layer "B.Cu") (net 19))
 (segment (start 79 39.24) (end 79 98.24) (width 1) (layer "B.Cu") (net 19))
 (segment (start 88 30.24) (end 79 39.24) (width 1) (layer "B.Cu") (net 19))
 (segment (start 91.88 88.86) (end 85.64 88.86) (width 1) (layer "B.Cu") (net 14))
 (segment (start 95 85.74) (end 91.88 88.86) (width 1) (layer "B.Cu") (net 14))
 (segment (start 112.96 32.78) (end 95 50.74) (width 1) (layer "B.Cu") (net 14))
 (segment (start 95 50.74) (end 95 85.74) (width 1) (layer "B.Cu") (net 14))
 (segment (start 123.5 32.78) (end 112.96 32.78) (width 1) (layer "B.Cu") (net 14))
 (segment (start 91 86.24) (end 101 96.24) (width 1) (layer "F.Cu") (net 4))
 (segment (start 101 96.24) (end 101 97.24) (width 1) (layer "F.Cu") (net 4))
 (via (at 101 97.24) (size 2) (drill 0.8) (layers "F.Cu" "B.Cu") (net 4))
 (via (at 91 86.24) (size 2) (drill 0.8) (layers "F.Cu" "B.Cu") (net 4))
 (segment (start 87.5 76.24) (end 91 79.74) (width 1) (layer "B.Cu") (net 4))
 (segment (start 101 115.74) (end 101 97.24) (width 1) (layer "B.Cu") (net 4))
 (segment (start 112 80.24) (end 112 80.74) (width 1) (layer "B.Cu") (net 4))
 (segment (start 112 80.74) (end 112 115.24) (width 1) (layer "B.Cu") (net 4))
 (segment (start 85.64 76.16) (end 87.42 76.16) (width 1) (layer "B.Cu") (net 4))
 (segment (start 114.5 77.74) (end 112 80.24) (width 1) (layer "B.Cu") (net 4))
 (segment (start 103.5 118.24) (end 101 115.74) (width 1) (layer "B.Cu") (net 4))
 (segment (start 91 79.74) (end 91 86.24) (width 1) (layer "B.Cu") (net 4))
 (segment (start 109 118.24) (end 106 118.24) (width 1) (layer "B.Cu") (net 4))
 (segment (start 118 77.74) (end 114.5 77.74) (width 1) (layer "B.Cu") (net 4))
 (segment (start 106 118.24) (end 103.5 118.24) (width 1) (layer "B.Cu") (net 4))
 (segment (start 87.42 76.16) (end 87.5 76.24) (width 1) (layer "B.Cu") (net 4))
 (segment (start 112 115.24) (end 109 118.24) (width 1) (layer "B.Cu") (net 4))
 (segment (start 103.5 68.24) (end 93 68.24) (width 1) (layer "F.Cu") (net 9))
 (via (at 103.5 68.24) (size 2) (drill 0.8) (layers "F.Cu" "B.Cu") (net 9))
 (via (at 93 68.24) (size 2) (drill 0.8) (layers "F.Cu" "B.Cu") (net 9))
 (segment (start 107.5 53.74) (end 103.5 57.74) (width 1) (layer "B.Cu") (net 9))
 (segment (start 92.5 68.24) (end 93 68.24) (width 1) (layer "B.Cu") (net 9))
 (segment (start 103.5 57.74) (end 103.5 68.24) (width 1) (layer "B.Cu") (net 9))
 (segment (start 87.5 73.24) (end 92.5 68.24) (width 1) (layer "B.Cu") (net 9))
 (segment (start 121.5 53.74) (end 107.5 53.74) (width 1) (layer "B.Cu") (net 9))
 (segment (start 132.5 64.74) (end 121.5 53.74) (width 1) (layer "B.Cu") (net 9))
 (segment (start 85.64 73.62) (end 87.12 73.62) (width 1) (layer "B.Cu") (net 9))
 (segment (start 129.75 88.49) (end 132.5 85.74) (width 1) (layer "B.Cu") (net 9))
 (segment (start 87.12 73.62) (end 87.5 73.24) (width 1) (layer "B.Cu") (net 9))
 (segment (start 132.5 85.74) (end 132.5 64.74) (width 1) (layer "B.Cu") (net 9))
 (segment (start 73.8 68.54) (end 73.5 68.24) (width 1) (layer "F.Cu") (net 1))
 (segment (start 81.3 68.54) (end 73.8 68.54) (width 1) (layer "F.Cu") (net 1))
 (via (at 81.3 68.54) (size 2) (drill 0.8) (layers "F.Cu" "B.Cu") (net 1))
 (via (at 73.5 68.24) (size 2) (drill 0.8) (layers "F.Cu" "B.Cu") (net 1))
 (segment (start 49 79.24) (end 60 68.24) (width 1) (layer "B.Cu") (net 1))
 (segment (start 85.64 68.54) (end 81.3 68.54) (width 1) (layer "B.Cu") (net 1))
 (segment (start 49 87.74) (end 49 79.24) (width 1) (layer "B.Cu") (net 1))
 (segment (start 60 68.24) (end 73.5 68.24) (width 1) (layer "B.Cu") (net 1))
 (segment (start 72.25 70.99) (end 81.57 70.99) (width 1) (layer "F.Cu") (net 3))
 (segment (start 81.57 70.99) (end 81.66 71.08) (width 1) (layer "F.Cu") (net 3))
 (via (at 81.66 71.08) (size 2) (drill 0.8) (layers "F.Cu" "B.Cu") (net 3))
 (via (at 72.25 70.99) (size 2) (drill 0.8) (layers "F.Cu" "B.Cu") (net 3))
 (segment (start 72.25 87.99) (end 72.25 70.99) (width 1) (layer "B.Cu") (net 3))
 (segment (start 85.64 71.08) (end 81.66 71.08) (width 1) (layer "B.Cu") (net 3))
 (segment (start 82.25 97.49) (end 82.5 97.24) (width 1) (layer "F.Cu") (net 15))
 (segment (start 72.75 97.49) (end 82.25 97.49) (width 1) (layer "F.Cu") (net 15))
 (via (at 82.5 97.24) (size 2) (drill 0.8) (layers "F.Cu" "B.Cu") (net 15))
 (via (at 72.75 97.49) (size 2) (drill 0.8) (layers "F.Cu" "B.Cu") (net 15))
 (segment (start 84.34 91.4) (end 82.5 93.24) (width 1) (layer "B.Cu") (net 15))
 (segment (start 64.25 97.49) (end 72.75 97.49) (width 1) (layer "B.Cu") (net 15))
 (segment (start 82.5 93.24) (end 82.5 97.24) (width 1) (layer "B.Cu") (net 15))
 (segment (start 85.64 91.4) (end 84.34 91.4) (width 1) (layer "B.Cu") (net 15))
 (segment (start 102.5 92.24) (end 89 105.74) (width 1) (layer "B.Cu") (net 27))
 (segment (start 69 126.24) (end 52 109.24) (width 1) (layer "B.Cu") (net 27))
 (segment (start 52 84.74) (end 57.5 79.24) (width 1) (layer "B.Cu") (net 27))
 (segment (start 89 116.74) (end 79.5 126.24) (width 1) (layer "B.Cu") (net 27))
 (segment (start 52 109.24) (end 52 84.74) (width 1) (layer "B.Cu") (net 27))
 (segment (start 108.5 71.08) (end 105.66 71.08) (width 1) (layer "B.Cu") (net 27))
 (segment (start 102.5 74.24) (end 102.5 92.24) (width 1) (layer "B.Cu") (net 27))
 (segment (start 105.66 71.08) (end 102.5 74.24) (width 1) (layer "B.Cu") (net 27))
 (segment (start 79.5 126.24) (end 69 126.24) (width 1) (layer "B.Cu") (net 27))
 (segment (start 89 105.74) (end 89 116.74) (width 1) (layer "B.Cu") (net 27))
 (segment (start 85.64 111.72) (end 74.52 111.72) (width 1.5) (layer "B.Cu") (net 5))
 (segment (start 74.52 111.72) (end 73 113.24) (width 1.5) (layer "B.Cu") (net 5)))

